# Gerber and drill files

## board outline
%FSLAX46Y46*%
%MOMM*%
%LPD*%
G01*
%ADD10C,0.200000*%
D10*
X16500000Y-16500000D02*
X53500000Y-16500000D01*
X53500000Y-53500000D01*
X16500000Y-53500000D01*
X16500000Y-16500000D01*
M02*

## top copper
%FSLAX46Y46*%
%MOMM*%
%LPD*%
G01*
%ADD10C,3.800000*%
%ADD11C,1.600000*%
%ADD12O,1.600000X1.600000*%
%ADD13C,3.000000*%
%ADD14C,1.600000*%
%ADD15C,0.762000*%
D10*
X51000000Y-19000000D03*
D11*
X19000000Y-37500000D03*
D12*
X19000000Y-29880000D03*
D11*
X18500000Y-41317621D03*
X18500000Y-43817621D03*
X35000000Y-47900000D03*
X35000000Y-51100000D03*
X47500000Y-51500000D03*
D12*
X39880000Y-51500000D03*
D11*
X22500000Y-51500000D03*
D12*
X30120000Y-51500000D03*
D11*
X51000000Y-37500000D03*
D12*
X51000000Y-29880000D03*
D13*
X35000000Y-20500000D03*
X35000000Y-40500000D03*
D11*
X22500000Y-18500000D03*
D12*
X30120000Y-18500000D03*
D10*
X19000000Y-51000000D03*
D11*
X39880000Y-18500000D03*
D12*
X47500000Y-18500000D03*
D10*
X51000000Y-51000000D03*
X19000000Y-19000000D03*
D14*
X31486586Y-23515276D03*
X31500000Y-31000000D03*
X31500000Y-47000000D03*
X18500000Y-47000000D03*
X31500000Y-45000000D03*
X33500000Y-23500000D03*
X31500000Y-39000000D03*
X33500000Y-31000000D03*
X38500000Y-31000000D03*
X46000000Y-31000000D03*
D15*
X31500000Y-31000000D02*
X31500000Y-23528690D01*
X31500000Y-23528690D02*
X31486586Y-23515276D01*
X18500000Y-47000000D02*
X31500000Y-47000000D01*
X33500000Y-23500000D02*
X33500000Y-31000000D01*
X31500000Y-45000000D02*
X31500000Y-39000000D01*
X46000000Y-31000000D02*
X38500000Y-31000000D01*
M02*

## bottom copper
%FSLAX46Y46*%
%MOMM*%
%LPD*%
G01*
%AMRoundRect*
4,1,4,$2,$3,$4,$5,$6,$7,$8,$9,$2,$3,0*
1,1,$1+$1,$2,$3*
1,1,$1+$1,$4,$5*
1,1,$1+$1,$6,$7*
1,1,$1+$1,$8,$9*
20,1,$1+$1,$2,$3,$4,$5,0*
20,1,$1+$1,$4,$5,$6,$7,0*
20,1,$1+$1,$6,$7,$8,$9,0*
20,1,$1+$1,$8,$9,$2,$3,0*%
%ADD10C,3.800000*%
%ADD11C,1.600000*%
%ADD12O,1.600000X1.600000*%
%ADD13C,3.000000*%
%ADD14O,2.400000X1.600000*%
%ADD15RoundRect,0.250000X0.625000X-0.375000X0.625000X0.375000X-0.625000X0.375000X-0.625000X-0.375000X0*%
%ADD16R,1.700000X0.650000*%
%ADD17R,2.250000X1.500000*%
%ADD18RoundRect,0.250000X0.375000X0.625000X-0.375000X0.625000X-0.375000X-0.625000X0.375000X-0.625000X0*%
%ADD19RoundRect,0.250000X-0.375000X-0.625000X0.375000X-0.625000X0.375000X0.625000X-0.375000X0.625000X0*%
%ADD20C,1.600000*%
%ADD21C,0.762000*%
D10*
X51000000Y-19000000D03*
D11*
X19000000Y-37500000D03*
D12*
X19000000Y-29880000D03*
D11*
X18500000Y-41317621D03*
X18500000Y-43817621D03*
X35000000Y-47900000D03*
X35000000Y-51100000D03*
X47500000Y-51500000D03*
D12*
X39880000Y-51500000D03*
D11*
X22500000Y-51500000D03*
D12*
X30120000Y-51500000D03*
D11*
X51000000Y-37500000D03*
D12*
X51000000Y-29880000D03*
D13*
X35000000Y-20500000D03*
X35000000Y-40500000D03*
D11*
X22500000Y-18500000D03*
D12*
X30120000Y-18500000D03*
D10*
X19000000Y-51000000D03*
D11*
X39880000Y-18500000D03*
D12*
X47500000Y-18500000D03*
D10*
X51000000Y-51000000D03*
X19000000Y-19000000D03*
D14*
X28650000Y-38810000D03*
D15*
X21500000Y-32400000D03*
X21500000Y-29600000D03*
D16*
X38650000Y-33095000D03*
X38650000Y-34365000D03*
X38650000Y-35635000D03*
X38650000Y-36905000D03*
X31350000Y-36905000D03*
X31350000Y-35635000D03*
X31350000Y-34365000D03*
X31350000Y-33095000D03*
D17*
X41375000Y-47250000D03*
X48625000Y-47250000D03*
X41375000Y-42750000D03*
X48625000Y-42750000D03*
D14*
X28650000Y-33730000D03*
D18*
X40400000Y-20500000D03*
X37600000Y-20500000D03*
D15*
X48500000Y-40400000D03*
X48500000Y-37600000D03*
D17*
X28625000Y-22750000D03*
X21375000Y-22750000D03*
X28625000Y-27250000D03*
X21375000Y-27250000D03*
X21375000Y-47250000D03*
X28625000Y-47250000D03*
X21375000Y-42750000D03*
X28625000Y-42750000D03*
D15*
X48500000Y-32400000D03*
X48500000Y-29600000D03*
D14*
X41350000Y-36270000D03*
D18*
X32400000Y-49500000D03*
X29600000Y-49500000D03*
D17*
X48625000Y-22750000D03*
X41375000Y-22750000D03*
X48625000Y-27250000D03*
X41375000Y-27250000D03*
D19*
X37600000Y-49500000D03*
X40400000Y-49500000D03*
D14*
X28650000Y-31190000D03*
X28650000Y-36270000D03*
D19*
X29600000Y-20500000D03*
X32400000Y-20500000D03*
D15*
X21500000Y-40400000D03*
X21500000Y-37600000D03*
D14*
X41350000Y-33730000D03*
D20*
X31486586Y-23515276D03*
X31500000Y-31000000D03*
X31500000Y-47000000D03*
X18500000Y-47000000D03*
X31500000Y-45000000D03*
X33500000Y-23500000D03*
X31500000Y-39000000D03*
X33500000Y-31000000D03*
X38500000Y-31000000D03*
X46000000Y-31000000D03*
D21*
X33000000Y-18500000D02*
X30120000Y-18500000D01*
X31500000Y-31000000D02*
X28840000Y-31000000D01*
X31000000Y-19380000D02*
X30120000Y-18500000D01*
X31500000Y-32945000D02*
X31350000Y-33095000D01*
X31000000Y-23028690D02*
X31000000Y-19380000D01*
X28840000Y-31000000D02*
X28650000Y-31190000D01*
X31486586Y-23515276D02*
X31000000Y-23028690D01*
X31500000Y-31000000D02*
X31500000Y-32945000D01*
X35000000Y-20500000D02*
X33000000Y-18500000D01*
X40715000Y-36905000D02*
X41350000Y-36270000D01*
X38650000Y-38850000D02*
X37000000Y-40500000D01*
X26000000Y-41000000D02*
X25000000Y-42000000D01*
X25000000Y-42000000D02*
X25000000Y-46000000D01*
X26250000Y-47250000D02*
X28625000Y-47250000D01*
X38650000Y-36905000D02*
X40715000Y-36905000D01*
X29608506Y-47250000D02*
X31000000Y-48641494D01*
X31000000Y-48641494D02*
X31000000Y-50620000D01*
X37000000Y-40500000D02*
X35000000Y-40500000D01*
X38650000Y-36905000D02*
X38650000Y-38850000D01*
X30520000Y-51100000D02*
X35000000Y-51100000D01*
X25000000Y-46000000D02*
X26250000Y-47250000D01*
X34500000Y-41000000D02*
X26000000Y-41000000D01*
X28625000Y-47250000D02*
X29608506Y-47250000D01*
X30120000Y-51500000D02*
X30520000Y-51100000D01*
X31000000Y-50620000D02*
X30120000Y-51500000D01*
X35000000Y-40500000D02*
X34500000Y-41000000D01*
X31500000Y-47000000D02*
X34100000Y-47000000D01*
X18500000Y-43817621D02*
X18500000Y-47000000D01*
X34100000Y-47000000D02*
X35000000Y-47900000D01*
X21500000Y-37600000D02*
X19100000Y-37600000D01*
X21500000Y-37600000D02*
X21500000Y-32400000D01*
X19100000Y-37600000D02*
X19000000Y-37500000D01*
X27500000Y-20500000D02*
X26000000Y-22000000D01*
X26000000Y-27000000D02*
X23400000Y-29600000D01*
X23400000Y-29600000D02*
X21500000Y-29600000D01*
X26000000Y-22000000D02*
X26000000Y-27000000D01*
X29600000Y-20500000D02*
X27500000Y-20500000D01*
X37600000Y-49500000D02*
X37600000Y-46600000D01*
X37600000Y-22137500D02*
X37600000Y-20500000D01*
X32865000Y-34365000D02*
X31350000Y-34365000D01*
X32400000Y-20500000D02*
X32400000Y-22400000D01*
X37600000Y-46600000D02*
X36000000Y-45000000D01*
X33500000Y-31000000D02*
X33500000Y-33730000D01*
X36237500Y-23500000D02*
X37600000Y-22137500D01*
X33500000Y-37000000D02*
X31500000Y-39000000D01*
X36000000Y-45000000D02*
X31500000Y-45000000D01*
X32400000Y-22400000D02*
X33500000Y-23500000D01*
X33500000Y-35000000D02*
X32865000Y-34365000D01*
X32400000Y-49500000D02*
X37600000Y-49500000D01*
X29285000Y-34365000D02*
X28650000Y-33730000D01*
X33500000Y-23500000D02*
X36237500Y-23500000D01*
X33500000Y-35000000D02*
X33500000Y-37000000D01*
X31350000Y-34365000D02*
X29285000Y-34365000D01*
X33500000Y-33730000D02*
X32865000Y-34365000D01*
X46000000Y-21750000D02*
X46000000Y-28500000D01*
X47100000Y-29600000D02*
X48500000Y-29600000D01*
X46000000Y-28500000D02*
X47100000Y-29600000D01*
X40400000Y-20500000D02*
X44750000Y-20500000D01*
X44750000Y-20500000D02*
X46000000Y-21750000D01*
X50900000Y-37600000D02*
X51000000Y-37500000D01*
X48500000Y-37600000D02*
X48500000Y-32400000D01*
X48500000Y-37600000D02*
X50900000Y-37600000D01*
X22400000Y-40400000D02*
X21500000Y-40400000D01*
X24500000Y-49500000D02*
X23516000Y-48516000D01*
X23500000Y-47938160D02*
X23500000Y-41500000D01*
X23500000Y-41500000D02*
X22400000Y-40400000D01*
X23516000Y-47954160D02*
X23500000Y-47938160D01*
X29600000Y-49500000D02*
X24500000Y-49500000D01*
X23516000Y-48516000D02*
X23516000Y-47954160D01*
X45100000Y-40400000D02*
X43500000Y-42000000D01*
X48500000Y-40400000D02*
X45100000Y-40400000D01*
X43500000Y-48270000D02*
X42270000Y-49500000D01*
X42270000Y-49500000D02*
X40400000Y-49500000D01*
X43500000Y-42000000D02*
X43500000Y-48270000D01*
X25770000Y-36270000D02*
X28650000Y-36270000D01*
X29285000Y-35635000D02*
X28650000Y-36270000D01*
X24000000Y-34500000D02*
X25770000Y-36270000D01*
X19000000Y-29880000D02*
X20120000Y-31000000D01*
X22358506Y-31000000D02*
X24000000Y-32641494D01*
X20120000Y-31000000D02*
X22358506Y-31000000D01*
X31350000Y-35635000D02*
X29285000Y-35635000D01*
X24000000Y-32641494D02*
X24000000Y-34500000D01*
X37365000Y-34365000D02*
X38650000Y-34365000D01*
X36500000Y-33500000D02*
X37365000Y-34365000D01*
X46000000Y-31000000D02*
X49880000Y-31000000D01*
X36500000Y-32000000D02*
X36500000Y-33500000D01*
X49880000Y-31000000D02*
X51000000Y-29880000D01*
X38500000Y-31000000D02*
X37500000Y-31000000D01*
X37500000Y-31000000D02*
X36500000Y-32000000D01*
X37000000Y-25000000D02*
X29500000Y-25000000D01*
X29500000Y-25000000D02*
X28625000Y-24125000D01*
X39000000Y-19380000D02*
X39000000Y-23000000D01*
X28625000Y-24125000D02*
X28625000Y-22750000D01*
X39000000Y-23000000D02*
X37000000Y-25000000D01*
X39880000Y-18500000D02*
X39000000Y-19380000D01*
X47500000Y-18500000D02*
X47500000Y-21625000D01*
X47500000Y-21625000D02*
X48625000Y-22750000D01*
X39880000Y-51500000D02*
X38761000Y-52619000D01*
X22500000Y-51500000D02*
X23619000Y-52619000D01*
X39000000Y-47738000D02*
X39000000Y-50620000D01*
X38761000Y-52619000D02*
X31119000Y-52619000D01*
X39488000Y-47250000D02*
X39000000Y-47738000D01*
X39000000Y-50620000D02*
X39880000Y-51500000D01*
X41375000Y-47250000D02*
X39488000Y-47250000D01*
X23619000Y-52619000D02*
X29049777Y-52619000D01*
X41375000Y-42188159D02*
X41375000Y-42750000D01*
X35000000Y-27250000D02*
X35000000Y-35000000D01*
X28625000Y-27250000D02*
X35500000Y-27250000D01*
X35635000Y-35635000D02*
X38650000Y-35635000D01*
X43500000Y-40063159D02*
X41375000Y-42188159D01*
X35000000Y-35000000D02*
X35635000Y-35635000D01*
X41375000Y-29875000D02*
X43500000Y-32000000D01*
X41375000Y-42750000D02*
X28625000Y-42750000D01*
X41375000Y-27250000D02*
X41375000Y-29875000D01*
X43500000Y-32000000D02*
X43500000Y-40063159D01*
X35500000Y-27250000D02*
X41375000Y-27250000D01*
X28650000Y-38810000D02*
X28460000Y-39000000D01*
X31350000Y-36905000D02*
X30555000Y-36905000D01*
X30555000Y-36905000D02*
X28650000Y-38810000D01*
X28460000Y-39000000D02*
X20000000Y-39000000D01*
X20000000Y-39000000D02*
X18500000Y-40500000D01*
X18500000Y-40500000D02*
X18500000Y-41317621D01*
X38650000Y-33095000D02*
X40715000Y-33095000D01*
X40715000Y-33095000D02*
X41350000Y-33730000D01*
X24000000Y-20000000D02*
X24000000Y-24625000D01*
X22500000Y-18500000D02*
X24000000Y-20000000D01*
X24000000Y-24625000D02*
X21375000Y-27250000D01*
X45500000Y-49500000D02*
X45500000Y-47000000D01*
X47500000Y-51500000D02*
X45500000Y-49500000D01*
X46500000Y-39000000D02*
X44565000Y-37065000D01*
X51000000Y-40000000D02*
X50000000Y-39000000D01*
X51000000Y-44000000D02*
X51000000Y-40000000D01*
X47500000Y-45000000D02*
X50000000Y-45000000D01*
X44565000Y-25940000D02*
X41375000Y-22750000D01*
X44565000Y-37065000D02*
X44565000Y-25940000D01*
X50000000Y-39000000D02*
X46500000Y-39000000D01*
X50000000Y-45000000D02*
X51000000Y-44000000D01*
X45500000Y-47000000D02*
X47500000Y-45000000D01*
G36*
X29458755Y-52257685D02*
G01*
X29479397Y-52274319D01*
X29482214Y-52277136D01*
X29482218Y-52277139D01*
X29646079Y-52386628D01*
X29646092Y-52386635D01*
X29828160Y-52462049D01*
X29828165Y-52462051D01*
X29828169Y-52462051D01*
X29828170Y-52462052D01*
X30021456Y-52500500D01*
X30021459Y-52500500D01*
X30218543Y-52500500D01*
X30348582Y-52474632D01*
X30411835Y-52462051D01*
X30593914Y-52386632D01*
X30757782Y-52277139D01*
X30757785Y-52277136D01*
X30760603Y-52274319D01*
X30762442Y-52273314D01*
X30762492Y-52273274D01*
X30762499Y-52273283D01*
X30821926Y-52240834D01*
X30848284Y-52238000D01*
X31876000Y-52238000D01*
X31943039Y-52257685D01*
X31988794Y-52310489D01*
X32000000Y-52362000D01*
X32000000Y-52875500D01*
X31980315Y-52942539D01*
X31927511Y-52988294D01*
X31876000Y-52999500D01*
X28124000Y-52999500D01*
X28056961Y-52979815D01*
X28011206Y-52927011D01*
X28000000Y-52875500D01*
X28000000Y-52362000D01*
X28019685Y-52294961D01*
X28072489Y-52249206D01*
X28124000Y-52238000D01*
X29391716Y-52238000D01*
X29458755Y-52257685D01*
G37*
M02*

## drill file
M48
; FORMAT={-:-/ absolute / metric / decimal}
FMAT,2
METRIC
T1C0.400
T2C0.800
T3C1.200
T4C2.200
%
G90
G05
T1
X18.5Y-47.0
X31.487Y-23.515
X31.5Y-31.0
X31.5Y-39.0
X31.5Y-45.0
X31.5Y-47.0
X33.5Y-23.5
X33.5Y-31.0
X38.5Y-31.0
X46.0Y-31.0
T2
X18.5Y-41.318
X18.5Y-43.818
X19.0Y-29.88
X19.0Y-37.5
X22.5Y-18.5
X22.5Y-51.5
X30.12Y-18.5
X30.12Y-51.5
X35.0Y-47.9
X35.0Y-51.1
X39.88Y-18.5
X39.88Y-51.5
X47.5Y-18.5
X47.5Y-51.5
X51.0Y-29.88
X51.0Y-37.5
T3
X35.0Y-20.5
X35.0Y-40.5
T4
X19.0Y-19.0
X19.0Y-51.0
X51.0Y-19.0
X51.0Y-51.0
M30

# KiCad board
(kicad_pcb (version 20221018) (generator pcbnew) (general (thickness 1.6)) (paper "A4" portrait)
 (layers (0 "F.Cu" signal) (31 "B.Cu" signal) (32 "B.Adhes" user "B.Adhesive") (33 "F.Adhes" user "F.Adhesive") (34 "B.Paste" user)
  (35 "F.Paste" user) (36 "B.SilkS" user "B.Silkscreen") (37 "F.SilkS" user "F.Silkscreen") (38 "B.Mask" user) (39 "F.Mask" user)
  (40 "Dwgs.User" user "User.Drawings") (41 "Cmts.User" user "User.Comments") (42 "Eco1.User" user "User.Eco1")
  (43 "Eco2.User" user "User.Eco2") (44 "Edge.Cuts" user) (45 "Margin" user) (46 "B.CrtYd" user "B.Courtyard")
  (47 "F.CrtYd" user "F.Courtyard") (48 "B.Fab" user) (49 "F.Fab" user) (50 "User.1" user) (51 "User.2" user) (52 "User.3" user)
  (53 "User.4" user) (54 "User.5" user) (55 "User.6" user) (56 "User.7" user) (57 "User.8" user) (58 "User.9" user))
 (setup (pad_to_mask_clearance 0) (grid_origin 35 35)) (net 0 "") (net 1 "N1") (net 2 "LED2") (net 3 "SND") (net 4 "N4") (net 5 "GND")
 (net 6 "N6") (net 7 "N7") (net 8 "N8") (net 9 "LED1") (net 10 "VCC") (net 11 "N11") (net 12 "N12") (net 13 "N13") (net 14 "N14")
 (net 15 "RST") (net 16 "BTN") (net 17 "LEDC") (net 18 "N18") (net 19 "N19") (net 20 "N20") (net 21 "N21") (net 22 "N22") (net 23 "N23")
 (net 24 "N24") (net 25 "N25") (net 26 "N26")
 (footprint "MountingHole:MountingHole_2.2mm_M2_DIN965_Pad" (layer "F.Cu") (at 51 19)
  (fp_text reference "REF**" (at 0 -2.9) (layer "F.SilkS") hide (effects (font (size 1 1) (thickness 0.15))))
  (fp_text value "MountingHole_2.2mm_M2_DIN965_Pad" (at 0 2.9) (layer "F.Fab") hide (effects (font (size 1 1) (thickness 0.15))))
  (pad "1" thru_hole circle (at 0 0) (size 3.8 3.8) (drill 2.2) (layers "*.Cu" "*.Mask")))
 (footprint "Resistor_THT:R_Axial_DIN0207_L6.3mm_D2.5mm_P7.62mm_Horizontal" (layer "F.Cu") (at 19 37.5 90)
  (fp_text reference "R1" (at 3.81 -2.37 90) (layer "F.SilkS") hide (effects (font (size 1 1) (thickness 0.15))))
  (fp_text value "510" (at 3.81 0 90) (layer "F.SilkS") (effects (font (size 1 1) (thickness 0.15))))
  (pad "1" thru_hole circle (at 0 0 90) (size 1.6 1.6) (drill 0.8) (layers "*.Cu" "*.Mask") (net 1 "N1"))
  (pad "2" thru_hole oval (at 7.62 0 90) (size 1.6 1.6) (drill 0.8) (layers "*.Cu" "*.Mask") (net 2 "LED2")))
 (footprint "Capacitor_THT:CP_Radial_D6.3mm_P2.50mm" (layer "F.Cu") (at 18.5 41.317621 -90)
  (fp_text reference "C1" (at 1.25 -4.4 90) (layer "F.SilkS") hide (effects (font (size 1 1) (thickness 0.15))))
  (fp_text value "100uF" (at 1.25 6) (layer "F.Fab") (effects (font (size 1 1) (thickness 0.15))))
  (pad "1" thru_hole circle (at 0 0 270) (size 1.6 1.6) (drill 0.8) (layers "*.Cu" "*.Mask") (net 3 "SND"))
  (pad "2" thru_hole circle (at 2.5 0 270) (size 1.6 1.6) (drill 0.8) (layers "*.Cu" "*.Mask") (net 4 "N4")))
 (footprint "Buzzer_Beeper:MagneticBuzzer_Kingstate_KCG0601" (layer "F.Cu") (at 35 47.9 -90)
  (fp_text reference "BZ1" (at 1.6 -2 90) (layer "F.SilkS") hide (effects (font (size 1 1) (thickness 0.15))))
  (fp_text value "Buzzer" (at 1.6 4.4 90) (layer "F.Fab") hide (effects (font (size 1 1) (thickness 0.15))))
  (pad "1" thru_hole circle (at 0 0 270) (size 1.6 1.6) (drill 0.8) (layers "*.Cu" "*.Mask") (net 4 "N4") (thermal_bridge_angle 90))
  (pad "2" thru_hole circle (at 3.2 0 270) (size 1.6 1.6) (drill 0.8) (layers "*.Cu" "*.Mask") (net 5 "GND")))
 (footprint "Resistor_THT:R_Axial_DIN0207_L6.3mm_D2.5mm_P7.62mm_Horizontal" (layer "F.Cu") (at 47.5 51.5 180)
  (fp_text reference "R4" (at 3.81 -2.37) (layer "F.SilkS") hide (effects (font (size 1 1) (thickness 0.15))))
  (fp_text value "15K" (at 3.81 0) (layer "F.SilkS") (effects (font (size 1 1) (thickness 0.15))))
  (pad "1" thru_hole circle (at 0 0 180) (size 1.6 1.6) (drill 0.8) (layers "*.Cu" "*.Mask") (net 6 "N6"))
  (pad "2" thru_hole oval (at 7.62 0 180) (size 1.6 1.6) (drill 0.8) (layers "*.Cu" "*.Mask") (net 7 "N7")))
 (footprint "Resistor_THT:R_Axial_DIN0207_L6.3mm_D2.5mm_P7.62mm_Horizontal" (layer "F.Cu") (at 22.5 51.5)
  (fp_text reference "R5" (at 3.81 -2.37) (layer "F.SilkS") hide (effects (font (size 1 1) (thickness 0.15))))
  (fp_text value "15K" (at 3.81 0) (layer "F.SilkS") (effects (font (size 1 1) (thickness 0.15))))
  (pad "1" thru_hole circle (at 0 0) (size 1.6 1.6) (drill 0.8) (layers "*.Cu" "*.Mask") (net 7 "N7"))
  (pad "2" thru_hole oval (at 7.62 0) (size 1.6 1.6) (drill 0.8) (layers "*.Cu" "*.Mask") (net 5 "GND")))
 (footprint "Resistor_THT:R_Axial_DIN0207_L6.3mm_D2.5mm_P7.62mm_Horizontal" (layer "F.Cu") (at 51 37.5 90)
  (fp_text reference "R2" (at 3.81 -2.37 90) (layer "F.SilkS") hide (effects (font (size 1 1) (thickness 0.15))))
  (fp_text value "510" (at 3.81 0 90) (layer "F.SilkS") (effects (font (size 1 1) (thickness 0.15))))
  (pad "1" thru_hole circle (at 0 0 90) (size 1.6 1.6) (drill 0.8) (layers "*.Cu" "*.Mask") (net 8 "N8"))
  (pad "2" thru_hole oval (at 7.62 0 90) (size 1.6 1.6) (drill 0.8) (layers "*.Cu" "*.Mask") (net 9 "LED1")))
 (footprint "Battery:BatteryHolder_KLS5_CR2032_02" (layer "F.Cu") (at 35 34 90)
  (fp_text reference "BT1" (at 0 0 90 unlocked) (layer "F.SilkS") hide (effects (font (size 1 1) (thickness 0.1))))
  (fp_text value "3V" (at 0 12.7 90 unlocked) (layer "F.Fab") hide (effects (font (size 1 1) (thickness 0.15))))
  (pad "1" thru_hole circle (at 13.5 0 90) (size 3 3) (drill 1.2) (layers "*.Cu" "*.Mask") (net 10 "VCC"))
  (pad "2" thru_hole circle (at -6.5 0 90) (size 3 3) (drill 1.2) (layers "*.Cu" "*.Mask") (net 5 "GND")))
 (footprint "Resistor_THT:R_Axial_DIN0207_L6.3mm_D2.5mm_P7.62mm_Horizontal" (layer "F.Cu") (at 22.5 18.5)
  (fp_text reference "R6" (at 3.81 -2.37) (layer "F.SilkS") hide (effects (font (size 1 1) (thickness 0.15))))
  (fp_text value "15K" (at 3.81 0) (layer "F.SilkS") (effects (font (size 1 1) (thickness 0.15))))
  (pad "1" thru_hole circle (at 0 0) (size 1.6 1.6) (drill 0.8) (layers "*.Cu" "*.Mask") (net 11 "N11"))
  (pad "2" thru_hole oval (at 7.62 0) (size 1.6 1.6) (drill 0.8) (layers "*.Cu" "*.Mask") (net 10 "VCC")))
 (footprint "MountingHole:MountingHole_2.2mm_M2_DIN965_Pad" (layer "F.Cu") (at 19 51)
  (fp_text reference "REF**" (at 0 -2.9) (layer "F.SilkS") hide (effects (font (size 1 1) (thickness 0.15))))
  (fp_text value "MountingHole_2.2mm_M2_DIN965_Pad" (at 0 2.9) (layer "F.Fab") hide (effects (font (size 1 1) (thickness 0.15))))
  (pad "1" thru_hole circle (at 0 0) (size 3.8 3.8) (drill 2.2) (layers "*.Cu" "*.Mask")))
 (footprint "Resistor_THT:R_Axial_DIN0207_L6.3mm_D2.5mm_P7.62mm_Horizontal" (layer "F.Cu") (at 39.88 18.5)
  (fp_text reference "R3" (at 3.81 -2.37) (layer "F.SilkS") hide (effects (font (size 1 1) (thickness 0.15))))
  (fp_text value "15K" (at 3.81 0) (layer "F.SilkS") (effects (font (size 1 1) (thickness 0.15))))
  (pad "1" thru_hole circle (at 0 0) (size 1.6 1.6) (drill 0.8) (layers "*.Cu" "*.Mask") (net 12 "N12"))
  (pad "2" thru_hole oval (at 7.62 0) (size 1.6 1.6) (drill 0.8) (layers "*.Cu" "*.Mask") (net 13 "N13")))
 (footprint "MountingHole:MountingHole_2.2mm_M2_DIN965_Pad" (layer "F.Cu") (at 51 51)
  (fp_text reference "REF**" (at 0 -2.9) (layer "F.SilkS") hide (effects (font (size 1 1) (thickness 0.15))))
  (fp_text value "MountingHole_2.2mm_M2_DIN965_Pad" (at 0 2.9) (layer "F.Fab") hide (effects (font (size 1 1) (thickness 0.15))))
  (pad "1" thru_hole circle (at 0 0) (size 3.8 3.8) (drill 2.2) (layers "*.Cu" "*.Mask")))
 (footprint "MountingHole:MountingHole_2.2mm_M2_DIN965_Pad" (layer "F.Cu") (at 19 19)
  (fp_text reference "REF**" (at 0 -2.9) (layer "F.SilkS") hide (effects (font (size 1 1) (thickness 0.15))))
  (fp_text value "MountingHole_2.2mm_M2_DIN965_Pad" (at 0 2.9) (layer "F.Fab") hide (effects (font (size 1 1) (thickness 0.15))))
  (pad "1" thru_hole circle (at 0 0) (size 3.8 3.8) (drill 2.2) (layers "*.Cu" "*.Mask")))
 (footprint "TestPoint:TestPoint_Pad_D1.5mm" (layer "B.Cu") (at 28.65 38.81 180)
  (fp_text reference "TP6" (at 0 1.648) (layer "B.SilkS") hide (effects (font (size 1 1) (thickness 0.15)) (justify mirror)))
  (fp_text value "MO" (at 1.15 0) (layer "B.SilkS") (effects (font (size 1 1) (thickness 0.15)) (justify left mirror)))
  (pad "1" smd oval (at 0 0 180) (size 2.4 1.6) (layers "B.Cu" "B.Mask") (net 3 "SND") (thermal_bridge_angle 45)))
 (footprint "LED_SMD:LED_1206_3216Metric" (layer "B.Cu") (at 21.5 31 90)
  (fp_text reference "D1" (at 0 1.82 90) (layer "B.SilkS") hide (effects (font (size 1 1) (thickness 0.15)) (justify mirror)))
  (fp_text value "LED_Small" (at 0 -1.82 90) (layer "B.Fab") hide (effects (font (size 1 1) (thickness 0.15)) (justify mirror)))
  (pad "1" smd roundrect (at -1.4 0 90) (size 1.25 1.75) (layers "B.Cu" "B.Paste" "B.Mask") (roundrect_rratio 0.2) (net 1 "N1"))
  (pad "2" smd roundrect (at 1.4 0 90) (size 1.25 1.75) (layers "B.Cu" "B.Paste" "B.Mask") (roundrect_rratio 0.2) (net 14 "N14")))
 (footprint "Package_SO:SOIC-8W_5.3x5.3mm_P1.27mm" (layer "B.Cu") (at 35 35 180)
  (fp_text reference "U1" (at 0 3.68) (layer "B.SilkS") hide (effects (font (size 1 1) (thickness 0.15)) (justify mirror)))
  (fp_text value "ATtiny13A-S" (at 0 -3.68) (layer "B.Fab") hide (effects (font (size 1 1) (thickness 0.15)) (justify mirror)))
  (pad "1" smd rect (at -3.65 1.905 180) (size 1.7 0.65) (layers "B.Cu" "B.Paste" "B.Mask") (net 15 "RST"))
  (pad "2" smd rect (at -3.65 0.635 180) (size 1.7 0.65) (layers "B.Cu" "B.Paste" "B.Mask") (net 9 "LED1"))
  (pad "3" smd rect (at -3.65 -0.635 180) (size 1.7 0.65) (layers "B.Cu" "B.Paste" "B.Mask") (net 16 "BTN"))
  (pad "4" smd rect (at -3.65 -1.905 180) (size 1.7 0.65) (layers "B.Cu" "B.Paste" "B.Mask") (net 5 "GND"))
  (pad "5" smd rect (at 3.65 -1.905 180) (size 1.7 0.65) (layers "B.Cu" "B.Paste" "B.Mask") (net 3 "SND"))
  (pad "6" smd rect (at 3.65 -0.635 180) (size 1.7 0.65) (layers "B.Cu" "B.Paste" "B.Mask") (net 2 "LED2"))
  (pad "7" smd rect (at 3.65 0.635 180) (size 1.7 0.65) (layers "B.Cu" "B.Paste" "B.Mask") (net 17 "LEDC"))
  (pad "8" smd rect (at 3.65 1.905 180) (size 1.7 0.65) (layers "B.Cu" "B.Paste" "B.Mask") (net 10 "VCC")))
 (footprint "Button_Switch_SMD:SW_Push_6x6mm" (layer "B.Cu") (at 45 45)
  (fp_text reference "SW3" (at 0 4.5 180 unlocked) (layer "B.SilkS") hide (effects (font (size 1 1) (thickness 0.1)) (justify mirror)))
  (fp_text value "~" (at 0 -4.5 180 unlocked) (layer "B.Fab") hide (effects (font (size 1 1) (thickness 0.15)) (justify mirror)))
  (pad "1" smd rect (at -3.625 2.25) (size 2.25 1.5) (layers "B.Cu" "B.Paste" "B.Mask") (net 7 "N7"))
  (pad "2" smd rect (at 3.625 2.25) (size 2.25 1.5) (layers "B.Cu" "B.Paste" "B.Mask") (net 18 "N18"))
  (pad "3" smd rect (at -3.625 -2.25) (size 2.25 1.5) (layers "B.Cu" "B.Paste" "B.Mask") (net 16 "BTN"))
  (pad "4" smd rect (at 3.625 -2.25) (size 2.25 1.5) (layers "B.Cu" "B.Paste" "B.Mask") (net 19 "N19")))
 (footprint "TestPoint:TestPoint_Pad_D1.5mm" (layer "B.Cu") (at 28.65 33.73 180)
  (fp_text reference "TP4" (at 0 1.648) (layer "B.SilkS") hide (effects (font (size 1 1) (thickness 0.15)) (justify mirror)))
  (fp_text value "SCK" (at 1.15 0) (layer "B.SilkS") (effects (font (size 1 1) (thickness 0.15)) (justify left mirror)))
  (pad "1" smd oval (at 0 0 180) (size 2.4 1.6) (layers "B.Cu" "B.Mask") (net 17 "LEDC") (thermal_bridge_angle 45)))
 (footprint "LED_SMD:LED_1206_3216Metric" (layer "B.Cu") (at 39 20.5 180)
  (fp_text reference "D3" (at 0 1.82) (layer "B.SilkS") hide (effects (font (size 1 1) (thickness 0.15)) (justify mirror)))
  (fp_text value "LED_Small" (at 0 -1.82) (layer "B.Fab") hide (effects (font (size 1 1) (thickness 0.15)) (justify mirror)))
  (pad "1" smd roundrect (at -1.4 0 180) (size 1.25 1.75) (layers "B.Cu" "B.Paste" "B.Mask") (roundrect_rratio 0.2) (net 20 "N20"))
  (pad "2" smd roundrect (at 1.4 0 180) (size 1.25 1.75) (layers "B.Cu" "B.Paste" "B.Mask") (roundrect_rratio 0.2) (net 17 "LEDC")))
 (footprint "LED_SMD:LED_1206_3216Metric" (layer "B.Cu") (at 48.5 39 90)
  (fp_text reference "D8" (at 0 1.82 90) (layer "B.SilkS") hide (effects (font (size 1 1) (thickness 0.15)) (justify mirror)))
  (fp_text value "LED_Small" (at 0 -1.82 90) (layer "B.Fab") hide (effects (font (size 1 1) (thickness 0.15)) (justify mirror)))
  (pad "1" smd roundrect (at -1.4 0 90) (size 1.25 1.75) (layers "B.Cu" "B.Paste" "B.Mask") (roundrect_rratio 0.2) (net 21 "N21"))
  (pad "2" smd roundrect (at 1.4 0 90) (size 1.25 1.75) (layers "B.Cu" "B.Paste" "B.Mask") (roundrect_rratio 0.2) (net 8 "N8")))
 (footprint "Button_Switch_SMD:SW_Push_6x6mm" (layer "B.Cu") (at 25 25 180)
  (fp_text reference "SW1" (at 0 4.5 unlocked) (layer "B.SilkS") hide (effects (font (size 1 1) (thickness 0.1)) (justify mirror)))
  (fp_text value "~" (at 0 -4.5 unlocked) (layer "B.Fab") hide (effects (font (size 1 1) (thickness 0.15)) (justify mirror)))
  (pad "1" smd rect (at -3.625 2.25 180) (size 2.25 1.5) (layers "B.Cu" "B.Paste" "B.Mask") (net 12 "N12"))
  (pad "2" smd rect (at 3.625 2.25 180) (size 2.25 1.5) (layers "B.Cu" "B.Paste" "B.Mask") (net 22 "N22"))
  (pad "3" smd rect (at -3.625 -2.25 180) (size 2.25 1.5) (layers "B.Cu" "B.Paste" "B.Mask") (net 16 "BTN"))
  (pad "4" smd rect (at 3.625 -2.25 180) (size 2.25 1.5) (layers "B.Cu" "B.Paste" "B.Mask") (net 11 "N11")))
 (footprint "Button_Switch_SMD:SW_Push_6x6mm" (layer "B.Cu") (at 25 45)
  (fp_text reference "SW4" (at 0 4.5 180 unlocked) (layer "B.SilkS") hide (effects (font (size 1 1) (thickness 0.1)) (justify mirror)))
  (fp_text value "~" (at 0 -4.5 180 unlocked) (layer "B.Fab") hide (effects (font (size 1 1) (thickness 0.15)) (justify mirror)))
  (pad "1" smd rect (at -3.625 2.25) (size 2.25 1.5) (layers "B.Cu" "B.Paste" "B.Mask") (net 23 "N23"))
  (pad "2" smd rect (at 3.625 2.25) (size 2.25 1.5) (layers "B.Cu" "B.Paste" "B.Mask") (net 5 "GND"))
  (pad "3" smd rect (at -3.625 -2.25) (size 2.25 1.5) (layers "B.Cu" "B.Paste" "B.Mask") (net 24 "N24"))
  (pad "4" smd rect (at 3.625 -2.25) (size 2.25 1.5) (layers "B.Cu" "B.Paste" "B.Mask") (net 16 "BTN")))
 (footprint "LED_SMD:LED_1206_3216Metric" (layer "B.Cu") (at 48.5 31 90)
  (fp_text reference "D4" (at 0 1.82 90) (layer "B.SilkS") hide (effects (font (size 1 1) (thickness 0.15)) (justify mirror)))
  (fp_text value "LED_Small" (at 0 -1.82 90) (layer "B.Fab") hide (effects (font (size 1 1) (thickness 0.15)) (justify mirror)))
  (pad "1" smd roundrect (at -1.4 0 90) (size 1.25 1.75) (layers "B.Cu" "B.Paste" "B.Mask") (roundrect_rratio 0.2) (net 8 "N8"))
  (pad "2" smd roundrect (at 1.4 0 90) (size 1.25 1.75) (layers "B.Cu" "B.Paste" "B.Mask") (roundrect_rratio 0.2) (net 20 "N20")))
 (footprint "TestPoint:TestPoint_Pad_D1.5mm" (layer "B.Cu") (at 41.35 36.27 180)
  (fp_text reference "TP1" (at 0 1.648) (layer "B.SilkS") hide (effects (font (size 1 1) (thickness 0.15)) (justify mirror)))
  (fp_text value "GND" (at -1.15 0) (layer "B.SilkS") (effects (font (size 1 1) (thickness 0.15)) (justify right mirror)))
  (pad "1" smd oval (at 0 0 180) (size 2.4 1.6) (layers "B.Cu" "B.Mask") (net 5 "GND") (thermal_bridge_angle 45)))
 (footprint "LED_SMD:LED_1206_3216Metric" (layer "B.Cu") (at 31 49.5 180)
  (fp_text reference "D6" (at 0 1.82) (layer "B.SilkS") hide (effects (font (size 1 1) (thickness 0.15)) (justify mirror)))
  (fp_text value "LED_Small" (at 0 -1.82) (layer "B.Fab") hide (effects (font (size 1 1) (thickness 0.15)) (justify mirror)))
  (pad "1" smd roundrect (at -1.4 0 180) (size 1.25 1.75) (layers "B.Cu" "B.Paste" "B.Mask") (roundrect_rratio 0.2) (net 17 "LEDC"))
  (pad "2" smd roundrect (at 1.4 0 180) (size 1.25 1.75) (layers "B.Cu" "B.Paste" "B.Mask") (roundrect_rratio 0.2) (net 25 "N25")))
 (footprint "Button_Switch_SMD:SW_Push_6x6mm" (layer "B.Cu") (at 45 25 180)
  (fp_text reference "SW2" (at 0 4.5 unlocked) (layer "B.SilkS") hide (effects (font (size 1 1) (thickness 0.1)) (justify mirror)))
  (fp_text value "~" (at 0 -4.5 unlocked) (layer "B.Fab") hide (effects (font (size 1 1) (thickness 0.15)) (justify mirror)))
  (pad "1" smd rect (at -3.625 2.25 180) (size 2.25 1.5) (layers "B.Cu" "B.Paste" "B.Mask") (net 13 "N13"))
  (pad "2" smd rect (at 3.625 2.25 180) (size 2.25 1.5) (layers "B.Cu" "B.Paste" "B.Mask") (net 6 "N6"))
  (pad "3" smd rect (at -3.625 -2.25 180) (size 2.25 1.5) (layers "B.Cu" "B.Paste" "B.Mask") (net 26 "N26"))
  (pad "4" smd rect (at 3.625 -2.25 180) (size 2.25 1.5) (layers "B.Cu" "B.Paste" "B.Mask") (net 16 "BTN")))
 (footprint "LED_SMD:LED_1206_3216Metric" (layer "B.Cu") (at 39 49.5)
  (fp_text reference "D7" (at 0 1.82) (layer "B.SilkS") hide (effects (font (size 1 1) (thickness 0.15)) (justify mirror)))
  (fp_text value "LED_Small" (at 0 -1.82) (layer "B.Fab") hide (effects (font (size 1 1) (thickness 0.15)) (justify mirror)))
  (pad "1" smd roundrect (at -1.4 0) (size 1.25 1.75) (layers "B.Cu" "B.Paste" "B.Mask") (roundrect_rratio 0.2) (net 17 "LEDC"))
  (pad "2" smd roundrect (at 1.4 0) (size 1.25 1.75) (layers "B.Cu" "B.Paste" "B.Mask") (roundrect_rratio 0.2) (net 21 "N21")))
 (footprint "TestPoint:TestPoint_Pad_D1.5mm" (layer "B.Cu") (at 28.65 31.19 180)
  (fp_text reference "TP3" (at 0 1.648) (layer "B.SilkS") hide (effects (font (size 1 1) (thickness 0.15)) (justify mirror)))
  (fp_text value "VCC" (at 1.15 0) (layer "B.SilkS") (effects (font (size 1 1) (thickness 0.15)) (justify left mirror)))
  (pad "1" smd oval (at 0 0 180) (size 2.4 1.6) (layers "B.Cu" "B.Mask") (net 10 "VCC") (thermal_bridge_angle 45)))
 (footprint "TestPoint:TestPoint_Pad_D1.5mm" (layer "B.Cu") (at 28.65 36.27 180)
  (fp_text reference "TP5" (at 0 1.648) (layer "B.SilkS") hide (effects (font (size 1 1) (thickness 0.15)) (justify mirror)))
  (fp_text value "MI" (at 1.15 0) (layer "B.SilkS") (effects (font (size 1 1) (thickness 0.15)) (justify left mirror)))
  (pad "1" smd oval (at 0 0 180) (size 2.4 1.6) (layers "B.Cu" "B.Mask") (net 2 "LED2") (thermal_bridge_angle 45)))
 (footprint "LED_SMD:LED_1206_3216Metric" (layer "B.Cu") (at 31 20.5)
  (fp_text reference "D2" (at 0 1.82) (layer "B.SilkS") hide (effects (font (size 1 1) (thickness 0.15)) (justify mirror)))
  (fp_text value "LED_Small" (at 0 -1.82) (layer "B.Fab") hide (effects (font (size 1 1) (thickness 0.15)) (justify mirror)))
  (pad "1" smd roundrect (at -1.4 0) (size 1.25 1.75) (layers "B.Cu" "B.Paste" "B.Mask") (roundrect_rratio 0.2) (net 14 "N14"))
  (pad "2" smd roundrect (at 1.4 0) (size 1.25 1.75) (layers "B.Cu" "B.Paste" "B.Mask") (roundrect_rratio 0.2) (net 17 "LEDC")))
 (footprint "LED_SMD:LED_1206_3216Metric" (layer "B.Cu") (at 21.5 39 90)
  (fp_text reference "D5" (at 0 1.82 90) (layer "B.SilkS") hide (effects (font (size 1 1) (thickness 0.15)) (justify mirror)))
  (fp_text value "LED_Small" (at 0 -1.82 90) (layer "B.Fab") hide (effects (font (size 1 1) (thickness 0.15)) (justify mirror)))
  (pad "1" smd roundrect (at -1.4 0 90) (size 1.25 1.75) (layers "B.Cu" "B.Paste" "B.Mask") (roundrect_rratio 0.2) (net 25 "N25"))
  (pad "2" smd roundrect (at 1.4 0 90) (size 1.25 1.75) (layers "B.Cu" "B.Paste" "B.Mask") (roundrect_rratio 0.2) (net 1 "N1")))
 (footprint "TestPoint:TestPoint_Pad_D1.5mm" (layer "B.Cu") (at 41.35 33.73 180)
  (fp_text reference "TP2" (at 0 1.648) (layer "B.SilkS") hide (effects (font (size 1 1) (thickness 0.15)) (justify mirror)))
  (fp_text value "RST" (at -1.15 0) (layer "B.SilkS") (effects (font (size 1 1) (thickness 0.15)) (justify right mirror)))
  (pad "1" smd oval (at 0 0 180) (size 2.4 1.6) (layers "B.Cu" "B.Mask") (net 15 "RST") (thermal_bridge_angle 45)))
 (gr_rect (start 16.5 16.5) (end 53.5 53.5) (stroke (width 0.2) (type default)) (fill none) (layer "Edge.Cuts"))
 (segment (start 31.5 31) (end 31.5 23.52869) (width 0.762) (layer "F.Cu") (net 10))
 (segment (start 31.5 23.52869) (end 31.486586 23.515276) (width 0.762) (layer "F.Cu") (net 10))
 (via (at 31.486586 23.515276) (size 1.6) (drill 0.4) (layers "F.Cu" "B.Cu") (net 10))
 (via (at 31.5 31) (size 1.6) (drill 0.4) (layers "F.Cu" "B.Cu") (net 10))
 (segment (start 33 18.5) (end 30.12 18.5) (width 0.762) (layer "B.Cu") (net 10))
 (segment (start 31.5 31) (end 28.84 31) (width 0.762) (layer "B.Cu") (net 10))
 (segment (start 31 19.38) (end 30.12 18.5) (width 0.762) (layer "B.Cu") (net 10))
 (segment (start 31.5 32.945) (end 31.35 33.095) (width 0.762) (layer "B.Cu") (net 10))
 (segment (start 31 23.02869) (end 31 19.38) (width 0.762) (layer "B.Cu") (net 10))
 (segment (start 28.84 31) (end 28.65 31.19) (width 0.762) (layer "B.Cu") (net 10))
 (segment (start 31.486586 23.515276) (end 31 23.02869) (width 0.762) (layer "B.Cu") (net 10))
 (segment (start 31.5 31) (end 31.5 32.945) (width 0.762) (layer "B.Cu") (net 10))
 (segment (start 35 20.5) (end 33 18.5) (width 0.762) (layer "B.Cu") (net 10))
 (segment (start 40.715 36.905) (end 41.35 36.27) (width 0.762) (layer "B.Cu") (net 5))
 (segment (start 38.65 38.85) (end 37 40.5) (width 0.762) (layer "B.Cu") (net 5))
 (segment (start 26 41) (end 25 42) (width 0.762) (layer "B.Cu") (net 5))
 (segment (start 25 42) (end 25 46) (width 0.762) (layer "B.Cu") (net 5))
 (segment (start 26.25 47.25) (end 28.625 47.25) (width 0.762) (layer "B.Cu") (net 5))
 (segment (start 38.65 36.905) (end 40.715 36.905) (width 0.762) (layer "B.Cu") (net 5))
 (segment (start 29.608506 47.25) (end 31 48.641494) (width 0.762) (layer "B.Cu") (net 5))
 (segment (start 31 48.641494) (end 31 50.62) (width 0.762) (layer "B.Cu") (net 5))
 (segment (start 37 40.5) (end 35 40.5) (width 0.762) (layer "B.Cu") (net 5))
 (segment (start 38.65 36.905) (end 38.65 38.85) (width 0.762) (layer "B.Cu") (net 5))
 (segment (start 30.52 51.1) (end 35 51.1) (width 0.762) (layer "B.Cu") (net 5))
 (segment (start 25 46) (end 26.25 47.25) (width 0.762) (layer "B.Cu") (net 5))
 (segment (start 34.5 41) (end 26 41) (width 0.762) (layer "B.Cu") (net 5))
 (segment (start 28.625 47.25) (end 29.608506 47.25) (width 0.762) (layer "B.Cu") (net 5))
 (segment (start 30.12 51.5) (end 30.52 51.1) (width 0.762) (layer "B.Cu") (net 5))
 (segment (start 31 50.62) (end 30.12 51.5) (width 0.762) (layer "B.Cu") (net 5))
 (segment (start 35 40.5) (end 34.5 41) (width 0.762) (layer "B.Cu") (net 5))
 (segment (start 18.5 47) (end 31.5 47) (width 0.762) (layer "F.Cu") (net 4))
 (via (at 31.5 47) (size 1.6) (drill 0.4) (layers "F.Cu" "B.Cu") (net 4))
 (via (at 18.5 47) (size 1.6) (drill 0.4) (layers "F.Cu" "B.Cu") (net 4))
 (segment (start 31.5 47) (end 34.1 47) (width 0.762) (layer "B.Cu") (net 4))
 (segment (start 18.5 43.817621) (end 18.5 47) (width 0.762) (layer "B.Cu") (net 4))
 (segment (start 34.1 47) (end 35 47.9) (width 0.762) (layer "B.Cu") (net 4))
 (segment (start 21.5 37.6) (end 19.1 37.6) (width 0.762) (layer "B.Cu") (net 1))
 (segment (start 21.5 37.6) (end 21.5 32.4) (width 0.762) (layer "B.Cu") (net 1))
 (segment (start 19.1 37.6) (end 19 37.5) (width 0.762) (layer "B.Cu") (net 1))
 (segment (start 27.5 20.5) (end 26 22) (width 0.762) (layer "B.Cu") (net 14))
 (segment (start 26 27) (end 23.4 29.6) (width 0.762) (layer "B.Cu") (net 14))
 (segment (start 23.4 29.6) (end 21.5 29.6) (width 0.762) (layer "B.Cu") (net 14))
 (segment (start 26 22) (end 26 27) (width 0.762) (layer "B.Cu") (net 14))
 (segment (start 29.6 20.5) (end 27.5 20.5) (width 0.762) (layer "B.Cu") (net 14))
 (segment (start 33.5 23.5) (end 33.5 31) (width 0.762) (layer "F.Cu") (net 17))
 (segment (start 31.5 45) (end 31.5 39) (width 0.762) (layer "F.Cu") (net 17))
 (via (at 31.5 45) (size 1.6) (drill 0.4) (layers "F.Cu" "B.Cu") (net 17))
 (via (at 33.5 23.5) (size 1.6) (drill 0.4) (layers "F.Cu" "B.Cu") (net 17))
 (via (at 31.5 39) (size 1.6) (drill 0.4) (layers "F.Cu" "B.Cu") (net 17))
 (via (at 33.5 31) (size 1.6) (drill 0.4) (layers "F.Cu" "B.Cu") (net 17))
 (segment (start 37.6 49.5) (end 37.6 46.6) (width 0.762) (layer "B.Cu") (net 17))
 (segment (start 37.6 22.1375) (end 37.6 20.5) (width 0.762) (layer "B.Cu") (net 17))
 (segment (start 32.865 34.365) (end 31.35 34.365) (width 0.762) (layer "B.Cu") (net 17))
 (segment (start 32.4 20.5) (end 32.4 22.4) (width 0.762) (layer "B.Cu") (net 17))
 (segment (start 37.6 46.6) (end 36 45) (width 0.762) (layer "B.Cu") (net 17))
 (segment (start 33.5 31) (end 33.5 33.73) (width 0.762) (layer "B.Cu") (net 17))
 (segment (start 36.2375 23.5) (end 37.6 22.1375) (width 0.762) (layer "B.Cu") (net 17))
 (segment (start 33.5 37) (end 31.5 39) (width 0.762) (layer "B.Cu") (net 17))
 (segment (start 36 45) (end 31.5 45) (width 0.762) (layer "B.Cu") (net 17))
 (segment (start 32.4 22.4) (end 33.5 23.5) (width 0.762) (layer "B.Cu") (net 17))
 (segment (start 33.5 35) (end 32.865 34.365) (width 0.762) (layer "B.Cu") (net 17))
 (segment (start 32.4 49.5) (end 37.6 49.5) (width 0.762) (layer "B.Cu") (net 17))
 (segment (start 29.285 34.365) (end 28.65 33.73) (width 0.762) (layer "B.Cu") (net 17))
 (segment (start 33.5 23.5) (end 36.2375 23.5) (width 0.762) (layer "B.Cu") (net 17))
 (segment (start 33.5 35) (end 33.5 37) (width 0.762) (layer "B.Cu") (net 17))
 (segment (start 31.35 34.365) (end 29.285 34.365) (width 0.762) (layer "B.Cu") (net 17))
 (segment (start 33.5 33.73) (end 32.865 34.365) (width 0.762) (layer "B.Cu") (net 17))
 (segment (start 46 21.75) (end 46 28.5) (width 0.762) (layer "B.Cu") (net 20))
 (segment (start 47.1 29.6) (end 48.5 29.6) (width 0.762) (layer "B.Cu") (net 20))
 (segment (start 46 28.5) (end 47.1 29.6) (width 0.762) (layer "B.Cu") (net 20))
 (segment (start 40.4 20.5) (end 44.75 20.5) (width 0.762) (layer "B.Cu") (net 20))
 (segment (start 44.75 20.5) (end 46 21.75) (width 0.762) (layer "B.Cu") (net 20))
 (segment (start 50.9 37.6) (end 51 37.5) (width 0.762) (layer "B.Cu") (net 8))
 (segment (start 48.5 37.6) (end 48.5 32.4) (width 0.762) (layer "B.Cu") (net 8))
 (segment (start 48.5 37.6) (end 50.9 37.6) (width 0.762) (layer "B.Cu") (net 8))
 (segment (start 22.4 40.4) (end 21.5 40.4) (width 0.762) (layer "B.Cu") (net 25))
 (segment (start 24.5 49.5) (end 23.516 48.516) (width 0.762) (layer "B.Cu") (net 25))
 (segment (start 23.5 47.93816) (end 23.5 41.5) (width 0.762) (layer "B.Cu") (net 25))
 (segment (start 23.5 41.5) (end 22.4 40.4) (width 0.762) (layer "B.Cu") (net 25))
 (segment (start 23.516 47.95416) (end 23.5 47.93816) (width 0.762) (layer "B.Cu") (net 25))
 (segment (start 29.6 49.5) (end 24.5 49.5) (width 0.762) (layer "B.Cu") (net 25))
 (segment (start 23.516 48.516) (end 23.516 47.95416) (width 0.762) (layer "B.Cu") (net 25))
 (segment (start 45.1 40.4) (end 43.5 42) (width 0.762) (layer "B.Cu") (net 21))
 (segment (start 48.5 40.4) (end 45.1 40.4) (width 0.762) (layer "B.Cu") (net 21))
 (segment (start 43.5 48.27) (end 42.27 49.5) (width 0.762) (layer "B.Cu") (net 21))
 (segment (start 42.27 49.5) (end 40.4 49.5) (width 0.762) (layer "B.Cu") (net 21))
 (segment (start 43.5 42) (end 43.5 48.27) (width 0.762) (layer "B.Cu") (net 21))
 (segment (start 25.77 36.27) (end 28.65 36.27) (width 0.762) (layer "B.Cu") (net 2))
 (segment (start 29.285 35.635) (end 28.65 36.27) (width 0.762) (layer "B.Cu") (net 2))
 (segment (start 24 34.5) (end 25.77 36.27) (width 0.762) (layer "B.Cu") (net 2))
 (segment (start 19 29.88) (end 20.12 31) (width 0.762) (layer "B.Cu") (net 2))
 (segment (start 22.358506 31) (end 24 32.641494) (width 0.762) (layer "B.Cu") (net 2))
 (segment (start 20.12 31) (end 22.358506 31) (width 0.762) (layer "B.Cu") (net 2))
 (segment (start 31.35 35.635) (end 29.285 35.635) (width 0.762) (layer "B.Cu") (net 2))
 (segment (start 24 32.641494) (end 24 34.5) (width 0.762) (layer "B.Cu") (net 2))
 (segment (start 46 31) (end 38.5 31) (width 0.762) (layer "F.Cu") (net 9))
 (via (at 38.5 31) (size 1.6) (drill 0.4) (layers "F.Cu" "B.Cu") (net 9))
 (via (at 46 31) (size 1.6) (drill 0.4) (layers "F.Cu" "B.Cu") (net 9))
 (segment (start 37.365 34.365) (end 38.65 34.365) (width 0.762) (layer "B.Cu") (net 9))
 (segment (start 36.5 33.5) (end 37.365 34.365) (width 0.762) (layer "B.Cu") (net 9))
 (segment (start 46 31) (end 49.88 31) (width 0.762) (layer "B.Cu") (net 9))
 (segment (start 36.5 32) (end 36.5 33.5) (width 0.762) (layer "B.Cu") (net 9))
 (segment (start 49.88 31) (end 51 29.88) (width 0.762) (layer "B.Cu") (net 9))
 (segment (start 38.5 31) (end 37.5 31) (width 0.762) (layer "B.Cu") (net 9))
 (segment (start 37.5 31) (end 36.5 32) (width 0.762) (layer "B.Cu") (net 9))
 (segment (start 37 25) (end 29.5 25) (width 0.762) (layer "B.Cu") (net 12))
 (segment (start 29.5 25) (end 28.625 24.125) (width 0.762) (layer "B.Cu") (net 12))
 (segment (start 39 19.38) (end 39 23) (width 0.762) (layer "B.Cu") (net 12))
 (segment (start 28.625 24.125) (end 28.625 22.75) (width 0.762) (layer "B.Cu") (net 12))
 (segment (start 39 23) (end 37 25) (width 0.762) (layer "B.Cu") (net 12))
 (segment (start 39.88 18.5) (end 39 19.38) (width 0.762) (layer "B.Cu") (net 12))
 (segment (start 47.5 18.5) (end 47.5 21.625) (width 0.762) (layer "B.Cu") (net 13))
 (segment (start 47.5 21.625) (end 48.625 22.75) (width 0.762) (layer "B.Cu") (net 13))
 (segment (start 39.88 51.5) (end 38.761 52.619) (width 0.762) (layer "B.Cu") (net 7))
 (segment (start 22.5 51.5) (end 23.619 52.619) (width 0.762) (layer "B.Cu") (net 7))
 (segment (start 39 47.738) (end 39 50.62) (width 0.762) (layer "B.Cu") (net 7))
 (segment (start 38.761 52.619) (end 31.119 52.619) (width 0.762) (layer "B.Cu") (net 7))
 (segment (start 39.488 47.25) (end 39 47.738) (width 0.762) (layer "B.Cu") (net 7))
 (segment (start 39 50.62) (end 39.88 51.5) (width 0.762) (layer "B.Cu") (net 7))
 (segment (start 41.375 47.25) (end 39.488 47.25) (width 0.762) (layer "B.Cu") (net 7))
 (segment (start 23.619 52.619) (end 29.049777 52.619) (width 0.762) (layer "B.Cu") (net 7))
 (segment (start 41.375 42.188159) (end 41.375 42.75) (width 0.762) (layer "B.Cu") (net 16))
 (segment (start 35 27.25) (end 35 35) (width 0.762) (layer "B.Cu") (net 16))
 (segment (start 28.625 27.25) (end 35.5 27.25) (width 0.762) (layer "B.Cu") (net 16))
 (segment (start 35.635 35.635) (end 38.65 35.635) (width 0.762) (layer "B.Cu") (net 16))
 (segment (start 43.5 40.063159) (end 41.375 42.188159) (width 0.762) (layer "B.Cu") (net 16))
 (segment (start 35 35) (end 35.635 35.635) (width 0.762) (layer "B.Cu") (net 16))
 (segment (start 41.375 29.875) (end 43.5 32) (width 0.762) (layer "B.Cu") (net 16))
 (segment (start 41.375 42.75) (end 28.625 42.75) (width 0.762) (layer "B.Cu") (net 16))
 (segment (start 41.375 27.25) (end 41.375 29.875) (width 0.762) (layer "B.Cu") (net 16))
 (segment (start 43.5 32) (end 43.5 40.063159) (width 0.762) (layer "B.Cu") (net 16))
 (segment (start 35.5 27.25) (end 41.375 27.25) (width 0.762) (layer "B.Cu") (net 16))
 (segment (start 28.65 38.81) (end 28.46 39) (width 0.762) (layer "B.Cu") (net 3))
 (segment (start 31.35 36.905) (end 30.555 36.905) (width 0.762) (layer "B.Cu") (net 3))
 (segment (start 30.555 36.905) (end 28.65 38.81) (width 0.762) (layer "B.Cu") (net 3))
 (segment (start 28.46 39) (end 20 39) (width 0.762) (layer "B.Cu") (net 3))
 (segment (start 20 39) (end 18.5 40.5) (width 0.762) (layer "B.Cu") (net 3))
 (segment (start 18.5 40.5) (end 18.5 41.317621) (width 0.762) (layer "B.Cu") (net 3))
 (segment (start 38.65 33.095) (end 40.715 33.095) (width 0.762) (layer "B.Cu") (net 15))
 (segment (start 40.715 33.095) (end 41.35 33.73) (width 0.762) (layer "B.Cu") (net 15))
 (segment (start 24 20) (end 24 24.625) (width 0.762) (layer "B.Cu") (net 11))
 (segment (start 22.5 18.5) (end 24 20) (width 0.762) (layer "B.Cu") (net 11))
 (segment (start 24 24.625) (end 21.375 27.25) (width 0.762) (layer "B.Cu") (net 11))
 (segment (start 45.5 49.5) (end 45.5 47) (width 0.762) (layer "B.Cu") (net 6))
 (segment (start 47.5 51.5) (end 45.5 49.5) (width 0.762) (layer "B.Cu") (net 6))
 (segment (start 46.5 39) (end 44.565 37.065) (width 0.762) (layer "B.Cu") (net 6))
 (segment (start 51 40) (end 50 39) (width 0.762) (layer "B.Cu") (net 6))
 (segment (start 51 44) (end 51 40) (width 0.762) (layer "B.Cu") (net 6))
 (segment (start 47.5 45) (end 50 45) (width 0.762) (layer "B.Cu") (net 6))
 (segment (start 44.565 25.94) (end 41.375 22.75) (width 0.762) (layer "B.Cu") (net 6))
 (segment (start 44.565 37.065) (end 44.565 25.94) (width 0.762) (layer "B.Cu") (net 6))
 (segment (start 50 39) (end 46.5 39) (width 0.762) (layer "B.Cu") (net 6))
 (segment (start 50 45) (end 51 44) (width 0.762) (layer "B.Cu") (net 6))
 (segment (start 45.5 47) (end 47.5 45) (width 0.762) (layer "B.Cu") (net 6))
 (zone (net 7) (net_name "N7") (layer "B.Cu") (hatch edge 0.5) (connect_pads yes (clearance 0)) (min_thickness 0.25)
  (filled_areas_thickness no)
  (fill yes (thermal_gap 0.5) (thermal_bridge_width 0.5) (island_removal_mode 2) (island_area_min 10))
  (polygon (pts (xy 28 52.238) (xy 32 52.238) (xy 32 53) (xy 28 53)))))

